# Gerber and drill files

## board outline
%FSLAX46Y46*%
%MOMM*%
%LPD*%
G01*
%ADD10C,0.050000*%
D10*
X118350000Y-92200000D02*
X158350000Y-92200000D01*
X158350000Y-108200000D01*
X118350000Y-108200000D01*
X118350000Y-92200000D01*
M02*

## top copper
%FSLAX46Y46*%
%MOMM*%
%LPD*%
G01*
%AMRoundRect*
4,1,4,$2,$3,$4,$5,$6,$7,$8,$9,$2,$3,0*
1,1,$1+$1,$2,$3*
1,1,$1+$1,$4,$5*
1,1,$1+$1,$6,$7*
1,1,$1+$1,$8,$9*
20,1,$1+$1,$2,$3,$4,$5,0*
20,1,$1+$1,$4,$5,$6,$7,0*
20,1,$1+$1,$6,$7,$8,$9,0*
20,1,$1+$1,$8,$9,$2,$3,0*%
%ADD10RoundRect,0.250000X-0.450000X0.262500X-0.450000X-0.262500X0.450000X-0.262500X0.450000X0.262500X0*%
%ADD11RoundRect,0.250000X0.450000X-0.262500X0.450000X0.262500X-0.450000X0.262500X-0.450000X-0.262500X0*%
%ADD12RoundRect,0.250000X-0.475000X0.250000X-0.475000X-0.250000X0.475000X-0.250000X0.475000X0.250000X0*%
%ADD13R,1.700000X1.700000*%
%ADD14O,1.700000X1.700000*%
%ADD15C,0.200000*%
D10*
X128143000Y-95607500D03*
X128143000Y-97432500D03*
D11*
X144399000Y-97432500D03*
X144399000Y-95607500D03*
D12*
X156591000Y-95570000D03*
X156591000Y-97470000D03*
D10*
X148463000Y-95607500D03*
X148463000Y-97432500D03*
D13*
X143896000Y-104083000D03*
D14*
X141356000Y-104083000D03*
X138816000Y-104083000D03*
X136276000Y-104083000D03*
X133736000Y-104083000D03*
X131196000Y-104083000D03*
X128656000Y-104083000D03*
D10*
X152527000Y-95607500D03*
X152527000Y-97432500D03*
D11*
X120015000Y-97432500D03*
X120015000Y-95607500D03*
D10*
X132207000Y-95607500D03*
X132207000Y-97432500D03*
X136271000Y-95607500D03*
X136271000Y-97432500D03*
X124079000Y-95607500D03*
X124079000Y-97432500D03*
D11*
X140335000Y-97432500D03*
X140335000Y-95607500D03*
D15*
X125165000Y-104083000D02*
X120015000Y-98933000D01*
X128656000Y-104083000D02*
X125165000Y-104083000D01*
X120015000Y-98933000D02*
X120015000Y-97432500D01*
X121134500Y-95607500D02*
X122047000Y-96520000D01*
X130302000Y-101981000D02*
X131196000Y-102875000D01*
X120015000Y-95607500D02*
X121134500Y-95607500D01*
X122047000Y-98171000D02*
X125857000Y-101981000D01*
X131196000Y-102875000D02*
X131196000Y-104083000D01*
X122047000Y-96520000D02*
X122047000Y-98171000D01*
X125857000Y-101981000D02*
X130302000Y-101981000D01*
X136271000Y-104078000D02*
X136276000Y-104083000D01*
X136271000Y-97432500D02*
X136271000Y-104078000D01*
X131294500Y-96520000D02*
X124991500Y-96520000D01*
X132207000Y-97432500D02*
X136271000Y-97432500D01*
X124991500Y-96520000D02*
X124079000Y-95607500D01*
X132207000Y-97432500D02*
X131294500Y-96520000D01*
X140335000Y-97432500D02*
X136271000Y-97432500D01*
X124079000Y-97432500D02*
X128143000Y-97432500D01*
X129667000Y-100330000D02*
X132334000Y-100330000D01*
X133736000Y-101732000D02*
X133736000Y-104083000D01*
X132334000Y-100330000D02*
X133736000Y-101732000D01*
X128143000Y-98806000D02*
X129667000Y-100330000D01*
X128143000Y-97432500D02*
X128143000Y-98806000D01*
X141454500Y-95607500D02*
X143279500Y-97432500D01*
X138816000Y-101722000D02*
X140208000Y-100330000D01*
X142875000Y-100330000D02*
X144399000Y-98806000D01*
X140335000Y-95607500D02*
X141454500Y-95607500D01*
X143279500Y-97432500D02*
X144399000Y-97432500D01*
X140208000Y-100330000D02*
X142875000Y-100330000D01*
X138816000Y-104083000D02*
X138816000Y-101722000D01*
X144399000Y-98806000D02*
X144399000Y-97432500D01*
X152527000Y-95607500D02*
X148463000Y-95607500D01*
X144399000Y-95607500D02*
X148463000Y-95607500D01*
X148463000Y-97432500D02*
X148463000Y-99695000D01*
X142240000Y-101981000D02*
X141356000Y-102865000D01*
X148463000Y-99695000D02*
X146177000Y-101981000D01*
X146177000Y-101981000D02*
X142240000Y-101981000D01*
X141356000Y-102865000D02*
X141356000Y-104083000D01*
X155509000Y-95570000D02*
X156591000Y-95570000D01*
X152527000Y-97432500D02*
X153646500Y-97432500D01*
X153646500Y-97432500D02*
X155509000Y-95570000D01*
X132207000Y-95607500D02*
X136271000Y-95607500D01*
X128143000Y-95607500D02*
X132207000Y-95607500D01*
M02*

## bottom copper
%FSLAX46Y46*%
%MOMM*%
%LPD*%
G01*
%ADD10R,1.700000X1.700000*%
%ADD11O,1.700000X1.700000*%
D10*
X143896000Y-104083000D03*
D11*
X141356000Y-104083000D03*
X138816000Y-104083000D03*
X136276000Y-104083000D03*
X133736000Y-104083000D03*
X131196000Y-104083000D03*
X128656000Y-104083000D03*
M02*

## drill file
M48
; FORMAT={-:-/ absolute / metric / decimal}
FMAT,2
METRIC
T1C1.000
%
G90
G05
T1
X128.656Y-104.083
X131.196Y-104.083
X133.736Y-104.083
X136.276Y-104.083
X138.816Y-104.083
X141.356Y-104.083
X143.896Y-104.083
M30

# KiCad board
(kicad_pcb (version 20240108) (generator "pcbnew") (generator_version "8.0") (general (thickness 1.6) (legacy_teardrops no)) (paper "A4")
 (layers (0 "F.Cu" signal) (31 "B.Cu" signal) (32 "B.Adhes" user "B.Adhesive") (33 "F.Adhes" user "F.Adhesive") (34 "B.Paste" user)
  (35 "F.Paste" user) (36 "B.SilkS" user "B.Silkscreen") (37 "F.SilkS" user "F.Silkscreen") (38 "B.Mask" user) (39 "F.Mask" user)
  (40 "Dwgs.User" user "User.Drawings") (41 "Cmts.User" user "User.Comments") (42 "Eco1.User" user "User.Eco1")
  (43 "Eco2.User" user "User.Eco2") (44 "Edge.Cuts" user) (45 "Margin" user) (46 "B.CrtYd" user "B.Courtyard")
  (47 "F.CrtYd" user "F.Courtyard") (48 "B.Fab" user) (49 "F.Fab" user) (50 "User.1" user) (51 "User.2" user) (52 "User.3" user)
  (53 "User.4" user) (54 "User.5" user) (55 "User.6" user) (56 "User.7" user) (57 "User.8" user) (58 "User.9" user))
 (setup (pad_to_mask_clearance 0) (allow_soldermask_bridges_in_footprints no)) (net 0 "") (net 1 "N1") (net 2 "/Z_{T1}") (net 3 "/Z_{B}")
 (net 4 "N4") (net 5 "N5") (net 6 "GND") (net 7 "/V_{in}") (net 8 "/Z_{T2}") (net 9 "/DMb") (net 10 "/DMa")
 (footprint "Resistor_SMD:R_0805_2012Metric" (layer "F.Cu") (at 128.143 96.52 -90)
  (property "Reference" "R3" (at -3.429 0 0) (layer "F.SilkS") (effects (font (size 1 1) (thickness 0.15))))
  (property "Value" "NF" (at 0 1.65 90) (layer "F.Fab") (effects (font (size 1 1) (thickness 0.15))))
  (pad "1" smd roundrect (at -0.9125 0 270) (size 1.025 1.4) (layers "F.Cu" "F.Paste" "F.Mask") (roundrect_rratio 0.243902) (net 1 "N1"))
  (pad "2" smd roundrect (at 0.9125 0 270) (size 1.025 1.4) (layers "F.Cu" "F.Paste" "F.Mask") (roundrect_rratio 0.243902) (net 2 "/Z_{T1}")))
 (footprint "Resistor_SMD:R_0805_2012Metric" (layer "F.Cu") (at 144.399 96.52 90)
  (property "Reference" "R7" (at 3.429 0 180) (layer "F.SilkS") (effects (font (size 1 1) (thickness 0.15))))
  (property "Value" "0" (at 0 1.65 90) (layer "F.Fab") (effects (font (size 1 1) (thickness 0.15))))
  (pad "1" smd roundrect (at -0.9125 0 90) (size 1.025 1.4) (layers "F.Cu" "F.Paste" "F.Mask") (roundrect_rratio 0.243902) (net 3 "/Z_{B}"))
  (pad "2" smd roundrect (at 0.9125 0 90) (size 1.025 1.4) (layers "F.Cu" "F.Paste" "F.Mask") (roundrect_rratio 0.243902) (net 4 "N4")))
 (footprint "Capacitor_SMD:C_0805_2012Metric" (layer "F.Cu") (at 156.591 96.52 -90)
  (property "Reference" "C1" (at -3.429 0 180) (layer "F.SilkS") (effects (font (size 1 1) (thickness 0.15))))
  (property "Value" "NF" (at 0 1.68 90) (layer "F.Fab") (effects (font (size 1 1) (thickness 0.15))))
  (pad "1" smd roundrect (at -0.95 0 270) (size 1 1.45) (layers "F.Cu" "F.Paste" "F.Mask") (roundrect_rratio 0.25) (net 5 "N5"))
  (pad "2" smd roundrect (at 0.95 0 270) (size 1 1.45) (layers "F.Cu" "F.Paste" "F.Mask") (roundrect_rratio 0.25) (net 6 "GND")))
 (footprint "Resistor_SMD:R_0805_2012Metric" (layer "F.Cu") (at 148.463 96.52 -90)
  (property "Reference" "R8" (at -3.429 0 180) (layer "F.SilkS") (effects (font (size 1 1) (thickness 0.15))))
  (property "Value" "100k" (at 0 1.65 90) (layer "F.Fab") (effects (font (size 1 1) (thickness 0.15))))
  (pad "1" smd roundrect (at -0.9125 0 270) (size 1.025 1.4) (layers "F.Cu" "F.Paste" "F.Mask") (roundrect_rratio 0.243902) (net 4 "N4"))
  (pad "2" smd roundrect (at 0.9125 0 270) (size 1.025 1.4) (layers "F.Cu" "F.Paste" "F.Mask") (roundrect_rratio 0.243902) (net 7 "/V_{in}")))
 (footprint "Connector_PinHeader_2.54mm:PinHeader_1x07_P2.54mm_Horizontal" (layer "F.Cu") (at 143.896 104.083 -90)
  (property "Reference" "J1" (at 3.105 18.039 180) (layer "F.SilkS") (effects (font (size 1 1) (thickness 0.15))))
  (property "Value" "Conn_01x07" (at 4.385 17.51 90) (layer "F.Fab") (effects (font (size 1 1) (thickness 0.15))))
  (pad "1" thru_hole rect (at 0 0 270) (size 1.7 1.7) (drill 1) (layers "*.Cu" "*.Mask") (remove_unused_layers no) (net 6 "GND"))
  (pad "2" thru_hole oval (at 0 2.54 270) (size 1.7 1.7) (drill 1) (layers "*.Cu" "*.Mask") (remove_unused_layers no) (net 7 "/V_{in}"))
  (pad "3" thru_hole oval (at 0 5.08 270) (size 1.7 1.7) (drill 1) (layers "*.Cu" "*.Mask") (remove_unused_layers no) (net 3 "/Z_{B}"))
  (pad "4" thru_hole oval (at 0 7.62 270) (size 1.7 1.7) (drill 1) (layers "*.Cu" "*.Mask") (remove_unused_layers no) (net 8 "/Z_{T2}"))
  (pad "5" thru_hole oval (at 0 10.16 270) (size 1.7 1.7) (drill 1) (layers "*.Cu" "*.Mask") (remove_unused_layers no) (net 2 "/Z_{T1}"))
  (pad "6" thru_hole oval (at 0 12.7 270) (size 1.7 1.7) (drill 1) (layers "*.Cu" "*.Mask") (remove_unused_layers no) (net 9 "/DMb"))
  (pad "7" thru_hole oval (at 0 15.24 270) (size 1.7 1.7) (drill 1) (layers "*.Cu" "*.Mask") (remove_unused_layers no) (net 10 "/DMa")))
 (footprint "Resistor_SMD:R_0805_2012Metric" (layer "F.Cu") (at 152.527 96.52 -90)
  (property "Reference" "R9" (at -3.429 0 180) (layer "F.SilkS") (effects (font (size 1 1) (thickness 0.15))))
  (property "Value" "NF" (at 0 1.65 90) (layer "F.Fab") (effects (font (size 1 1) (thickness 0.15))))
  (pad "1" smd roundrect (at -0.9125 0 270) (size 1.025 1.4) (layers "F.Cu" "F.Paste" "F.Mask") (roundrect_rratio 0.243902) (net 4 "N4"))
  (pad "2" smd roundrect (at 0.9125 0 270) (size 1.025 1.4) (layers "F.Cu" "F.Paste" "F.Mask") (roundrect_rratio 0.243902) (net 5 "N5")))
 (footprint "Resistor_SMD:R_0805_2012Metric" (layer "F.Cu") (at 120.015 96.52 90)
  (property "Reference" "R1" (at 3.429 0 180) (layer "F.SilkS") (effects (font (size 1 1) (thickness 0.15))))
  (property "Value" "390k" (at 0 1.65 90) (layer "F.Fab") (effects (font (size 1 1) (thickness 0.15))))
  (pad "1" smd roundrect (at -0.9125 0 90) (size 1.025 1.4) (layers "F.Cu" "F.Paste" "F.Mask") (roundrect_rratio 0.243902) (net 10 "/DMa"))
  (pad "2" smd roundrect (at 0.9125 0 90) (size 1.025 1.4) (layers "F.Cu" "F.Paste" "F.Mask") (roundrect_rratio 0.243902) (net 9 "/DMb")))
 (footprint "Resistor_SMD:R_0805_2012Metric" (layer "F.Cu") (at 132.207 96.52 -90)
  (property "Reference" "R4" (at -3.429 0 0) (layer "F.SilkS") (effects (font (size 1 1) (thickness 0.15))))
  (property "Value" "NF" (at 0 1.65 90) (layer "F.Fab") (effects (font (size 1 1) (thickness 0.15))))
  (pad "1" smd roundrect (at -0.9125 0 270) (size 1.025 1.4) (layers "F.Cu" "F.Paste" "F.Mask") (roundrect_rratio 0.243902) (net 1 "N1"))
  (pad "2" smd roundrect (at 0.9125 0 270) (size 1.025 1.4) (layers "F.Cu" "F.Paste" "F.Mask") (roundrect_rratio 0.243902) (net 8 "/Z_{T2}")))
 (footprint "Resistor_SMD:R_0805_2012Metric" (layer "F.Cu") (at 136.271 96.52 -90)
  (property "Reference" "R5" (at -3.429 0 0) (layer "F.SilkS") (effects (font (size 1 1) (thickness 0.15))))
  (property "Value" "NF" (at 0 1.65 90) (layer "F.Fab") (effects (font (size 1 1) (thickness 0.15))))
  (pad "1" smd roundrect (at -0.9125 0 270) (size 1.025 1.4) (layers "F.Cu" "F.Paste" "F.Mask") (roundrect_rratio 0.243902) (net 1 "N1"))
  (pad "2" smd roundrect (at 0.9125 0 270) (size 1.025 1.4) (layers "F.Cu" "F.Paste" "F.Mask") (roundrect_rratio 0.243902) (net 8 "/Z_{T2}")))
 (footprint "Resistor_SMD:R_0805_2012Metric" (layer "F.Cu") (at 124.079 96.52 -90)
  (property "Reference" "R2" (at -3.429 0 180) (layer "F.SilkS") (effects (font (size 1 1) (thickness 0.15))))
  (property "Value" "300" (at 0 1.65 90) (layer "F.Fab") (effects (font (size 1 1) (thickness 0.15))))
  (pad "1" smd roundrect (at -0.9125 0 270) (size 1.025 1.4) (layers "F.Cu" "F.Paste" "F.Mask") (roundrect_rratio 0.243902)
   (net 8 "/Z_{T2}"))
  (pad "2" smd roundrect (at 0.9125 0 270) (size 1.025 1.4) (layers "F.Cu" "F.Paste" "F.Mask") (roundrect_rratio 0.243902) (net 2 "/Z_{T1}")))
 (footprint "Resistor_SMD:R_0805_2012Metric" (layer "F.Cu") (at 140.335 96.52 90)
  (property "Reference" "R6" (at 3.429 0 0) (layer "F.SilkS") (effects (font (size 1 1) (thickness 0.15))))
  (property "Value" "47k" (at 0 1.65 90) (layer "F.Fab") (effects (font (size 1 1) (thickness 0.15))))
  (pad "1" smd roundrect (at -0.9125 0 90) (size 1.025 1.4) (layers "F.Cu" "F.Paste" "F.Mask") (roundrect_rratio 0.243902) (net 8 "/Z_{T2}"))
  (pad "2" smd roundrect (at 0.9125 0 90) (size 1.025 1.4) (layers "F.Cu" "F.Paste" "F.Mask") (roundrect_rratio 0.243902) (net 3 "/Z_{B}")))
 (gr_rect (start 118.35 92.2) (end 158.35 108.2) (stroke (width 0.05) (type default)) (fill none) (layer "Edge.Cuts"))
 (segment (start 125.165 104.083) (end 120.015 98.933) (width 0.2) (layer "F.Cu") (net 10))
 (segment (start 128.656 104.083) (end 125.165 104.083) (width 0.2) (layer "F.Cu") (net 10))
 (segment (start 120.015 98.933) (end 120.015 97.4325) (width 0.2) (layer "F.Cu") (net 10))
 (segment (start 121.1345 95.6075) (end 122.047 96.52) (width 0.2) (layer "F.Cu") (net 9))
 (segment (start 130.302 101.981) (end 131.196 102.875) (width 0.2) (layer "F.Cu") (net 9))
 (segment (start 120.015 95.6075) (end 121.1345 95.6075) (width 0.2) (layer "F.Cu") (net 9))
 (segment (start 122.047 98.171) (end 125.857 101.981) (width 0.2) (layer "F.Cu") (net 9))
 (segment (start 131.196 102.875) (end 131.196 104.083) (width 0.2) (layer "F.Cu") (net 9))
 (segment (start 122.047 96.52) (end 122.047 98.171) (width 0.2) (layer "F.Cu") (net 9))
 (segment (start 125.857 101.981) (end 130.302 101.981) (width 0.2) (layer "F.Cu") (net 9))
 (segment (start 136.271 104.078) (end 136.276 104.083) (width 0.2) (layer "F.Cu") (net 8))
 (segment (start 136.271 97.4325) (end 136.271 104.078) (width 0.2) (layer "F.Cu") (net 8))
 (segment (start 131.2945 96.52) (end 124.9915 96.52) (width 0.2) (layer "F.Cu") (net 8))
 (segment (start 132.207 97.4325) (end 136.271 97.4325) (width 0.2) (layer "F.Cu") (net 8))
 (segment (start 124.9915 96.52) (end 124.079 95.6075) (width 0.2) (layer "F.Cu") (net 8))
 (segment (start 132.207 97.4325) (end 131.2945 96.52) (width 0.2) (layer "F.Cu") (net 8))
 (segment (start 140.335 97.4325) (end 136.271 97.4325) (width 0.2) (layer "F.Cu") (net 8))
 (segment (start 124.079 97.4325) (end 128.143 97.4325) (width 0.2) (layer "F.Cu") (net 2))
 (segment (start 129.667 100.33) (end 132.334 100.33) (width 0.2) (layer "F.Cu") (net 2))
 (segment (start 133.736 101.732) (end 133.736 104.083) (width 0.2) (layer "F.Cu") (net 2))
 (segment (start 132.334 100.33) (end 133.736 101.732) (width 0.2) (layer "F.Cu") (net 2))
 (segment (start 128.143 98.806) (end 129.667 100.33) (width 0.2) (layer "F.Cu") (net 2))
 (segment (start 128.143 97.4325) (end 128.143 98.806) (width 0.2) (layer "F.Cu") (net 2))
 (segment (start 141.4545 95.6075) (end 143.2795 97.4325) (width 0.2) (layer "F.Cu") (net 3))
 (segment (start 138.816 101.722) (end 140.208 100.33) (width 0.2) (layer "F.Cu") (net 3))
 (segment (start 142.875 100.33) (end 144.399 98.806) (width 0.2) (layer "F.Cu") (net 3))
 (segment (start 140.335 95.6075) (end 141.4545 95.6075) (width 0.2) (layer "F.Cu") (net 3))
 (segment (start 143.2795 97.4325) (end 144.399 97.4325) (width 0.2) (layer "F.Cu") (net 3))
 (segment (start 140.208 100.33) (end 142.875 100.33) (width 0.2) (layer "F.Cu") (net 3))
 (segment (start 138.816 104.083) (end 138.816 101.722) (width 0.2) (layer "F.Cu") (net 3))
 (segment (start 144.399 98.806) (end 144.399 97.4325) (width 0.2) (layer "F.Cu") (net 3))
 (segment (start 152.527 95.6075) (end 148.463 95.6075) (width 0.2) (layer "F.Cu") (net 4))
 (segment (start 144.399 95.6075) (end 148.463 95.6075) (width 0.2) (layer "F.Cu") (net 4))
 (segment (start 148.463 97.4325) (end 148.463 99.695) (width 0.2) (layer "F.Cu") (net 7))
 (segment (start 142.24 101.981) (end 141.356 102.865) (width 0.2) (layer "F.Cu") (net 7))
 (segment (start 148.463 99.695) (end 146.177 101.981) (width 0.2) (layer "F.Cu") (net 7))
 (segment (start 146.177 101.981) (end 142.24 101.981) (width 0.2) (layer "F.Cu") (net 7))
 (segment (start 141.356 102.865) (end 141.356 104.083) (width 0.2) (layer "F.Cu") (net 7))
 (segment (start 155.509 95.57) (end 156.591 95.57) (width 0.2) (layer "F.Cu") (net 5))
 (segment (start 152.527 97.4325) (end 153.6465 97.4325) (width 0.2) (layer "F.Cu") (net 5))
 (segment (start 153.6465 97.4325) (end 155.509 95.57) (width 0.2) (layer "F.Cu") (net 5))
 (segment (start 132.207 95.6075) (end 136.271 95.6075) (width 0.2) (layer "F.Cu") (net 1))
 (segment (start 128.143 95.6075) (end 132.207 95.6075) (width 0.2) (layer "F.Cu") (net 1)))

